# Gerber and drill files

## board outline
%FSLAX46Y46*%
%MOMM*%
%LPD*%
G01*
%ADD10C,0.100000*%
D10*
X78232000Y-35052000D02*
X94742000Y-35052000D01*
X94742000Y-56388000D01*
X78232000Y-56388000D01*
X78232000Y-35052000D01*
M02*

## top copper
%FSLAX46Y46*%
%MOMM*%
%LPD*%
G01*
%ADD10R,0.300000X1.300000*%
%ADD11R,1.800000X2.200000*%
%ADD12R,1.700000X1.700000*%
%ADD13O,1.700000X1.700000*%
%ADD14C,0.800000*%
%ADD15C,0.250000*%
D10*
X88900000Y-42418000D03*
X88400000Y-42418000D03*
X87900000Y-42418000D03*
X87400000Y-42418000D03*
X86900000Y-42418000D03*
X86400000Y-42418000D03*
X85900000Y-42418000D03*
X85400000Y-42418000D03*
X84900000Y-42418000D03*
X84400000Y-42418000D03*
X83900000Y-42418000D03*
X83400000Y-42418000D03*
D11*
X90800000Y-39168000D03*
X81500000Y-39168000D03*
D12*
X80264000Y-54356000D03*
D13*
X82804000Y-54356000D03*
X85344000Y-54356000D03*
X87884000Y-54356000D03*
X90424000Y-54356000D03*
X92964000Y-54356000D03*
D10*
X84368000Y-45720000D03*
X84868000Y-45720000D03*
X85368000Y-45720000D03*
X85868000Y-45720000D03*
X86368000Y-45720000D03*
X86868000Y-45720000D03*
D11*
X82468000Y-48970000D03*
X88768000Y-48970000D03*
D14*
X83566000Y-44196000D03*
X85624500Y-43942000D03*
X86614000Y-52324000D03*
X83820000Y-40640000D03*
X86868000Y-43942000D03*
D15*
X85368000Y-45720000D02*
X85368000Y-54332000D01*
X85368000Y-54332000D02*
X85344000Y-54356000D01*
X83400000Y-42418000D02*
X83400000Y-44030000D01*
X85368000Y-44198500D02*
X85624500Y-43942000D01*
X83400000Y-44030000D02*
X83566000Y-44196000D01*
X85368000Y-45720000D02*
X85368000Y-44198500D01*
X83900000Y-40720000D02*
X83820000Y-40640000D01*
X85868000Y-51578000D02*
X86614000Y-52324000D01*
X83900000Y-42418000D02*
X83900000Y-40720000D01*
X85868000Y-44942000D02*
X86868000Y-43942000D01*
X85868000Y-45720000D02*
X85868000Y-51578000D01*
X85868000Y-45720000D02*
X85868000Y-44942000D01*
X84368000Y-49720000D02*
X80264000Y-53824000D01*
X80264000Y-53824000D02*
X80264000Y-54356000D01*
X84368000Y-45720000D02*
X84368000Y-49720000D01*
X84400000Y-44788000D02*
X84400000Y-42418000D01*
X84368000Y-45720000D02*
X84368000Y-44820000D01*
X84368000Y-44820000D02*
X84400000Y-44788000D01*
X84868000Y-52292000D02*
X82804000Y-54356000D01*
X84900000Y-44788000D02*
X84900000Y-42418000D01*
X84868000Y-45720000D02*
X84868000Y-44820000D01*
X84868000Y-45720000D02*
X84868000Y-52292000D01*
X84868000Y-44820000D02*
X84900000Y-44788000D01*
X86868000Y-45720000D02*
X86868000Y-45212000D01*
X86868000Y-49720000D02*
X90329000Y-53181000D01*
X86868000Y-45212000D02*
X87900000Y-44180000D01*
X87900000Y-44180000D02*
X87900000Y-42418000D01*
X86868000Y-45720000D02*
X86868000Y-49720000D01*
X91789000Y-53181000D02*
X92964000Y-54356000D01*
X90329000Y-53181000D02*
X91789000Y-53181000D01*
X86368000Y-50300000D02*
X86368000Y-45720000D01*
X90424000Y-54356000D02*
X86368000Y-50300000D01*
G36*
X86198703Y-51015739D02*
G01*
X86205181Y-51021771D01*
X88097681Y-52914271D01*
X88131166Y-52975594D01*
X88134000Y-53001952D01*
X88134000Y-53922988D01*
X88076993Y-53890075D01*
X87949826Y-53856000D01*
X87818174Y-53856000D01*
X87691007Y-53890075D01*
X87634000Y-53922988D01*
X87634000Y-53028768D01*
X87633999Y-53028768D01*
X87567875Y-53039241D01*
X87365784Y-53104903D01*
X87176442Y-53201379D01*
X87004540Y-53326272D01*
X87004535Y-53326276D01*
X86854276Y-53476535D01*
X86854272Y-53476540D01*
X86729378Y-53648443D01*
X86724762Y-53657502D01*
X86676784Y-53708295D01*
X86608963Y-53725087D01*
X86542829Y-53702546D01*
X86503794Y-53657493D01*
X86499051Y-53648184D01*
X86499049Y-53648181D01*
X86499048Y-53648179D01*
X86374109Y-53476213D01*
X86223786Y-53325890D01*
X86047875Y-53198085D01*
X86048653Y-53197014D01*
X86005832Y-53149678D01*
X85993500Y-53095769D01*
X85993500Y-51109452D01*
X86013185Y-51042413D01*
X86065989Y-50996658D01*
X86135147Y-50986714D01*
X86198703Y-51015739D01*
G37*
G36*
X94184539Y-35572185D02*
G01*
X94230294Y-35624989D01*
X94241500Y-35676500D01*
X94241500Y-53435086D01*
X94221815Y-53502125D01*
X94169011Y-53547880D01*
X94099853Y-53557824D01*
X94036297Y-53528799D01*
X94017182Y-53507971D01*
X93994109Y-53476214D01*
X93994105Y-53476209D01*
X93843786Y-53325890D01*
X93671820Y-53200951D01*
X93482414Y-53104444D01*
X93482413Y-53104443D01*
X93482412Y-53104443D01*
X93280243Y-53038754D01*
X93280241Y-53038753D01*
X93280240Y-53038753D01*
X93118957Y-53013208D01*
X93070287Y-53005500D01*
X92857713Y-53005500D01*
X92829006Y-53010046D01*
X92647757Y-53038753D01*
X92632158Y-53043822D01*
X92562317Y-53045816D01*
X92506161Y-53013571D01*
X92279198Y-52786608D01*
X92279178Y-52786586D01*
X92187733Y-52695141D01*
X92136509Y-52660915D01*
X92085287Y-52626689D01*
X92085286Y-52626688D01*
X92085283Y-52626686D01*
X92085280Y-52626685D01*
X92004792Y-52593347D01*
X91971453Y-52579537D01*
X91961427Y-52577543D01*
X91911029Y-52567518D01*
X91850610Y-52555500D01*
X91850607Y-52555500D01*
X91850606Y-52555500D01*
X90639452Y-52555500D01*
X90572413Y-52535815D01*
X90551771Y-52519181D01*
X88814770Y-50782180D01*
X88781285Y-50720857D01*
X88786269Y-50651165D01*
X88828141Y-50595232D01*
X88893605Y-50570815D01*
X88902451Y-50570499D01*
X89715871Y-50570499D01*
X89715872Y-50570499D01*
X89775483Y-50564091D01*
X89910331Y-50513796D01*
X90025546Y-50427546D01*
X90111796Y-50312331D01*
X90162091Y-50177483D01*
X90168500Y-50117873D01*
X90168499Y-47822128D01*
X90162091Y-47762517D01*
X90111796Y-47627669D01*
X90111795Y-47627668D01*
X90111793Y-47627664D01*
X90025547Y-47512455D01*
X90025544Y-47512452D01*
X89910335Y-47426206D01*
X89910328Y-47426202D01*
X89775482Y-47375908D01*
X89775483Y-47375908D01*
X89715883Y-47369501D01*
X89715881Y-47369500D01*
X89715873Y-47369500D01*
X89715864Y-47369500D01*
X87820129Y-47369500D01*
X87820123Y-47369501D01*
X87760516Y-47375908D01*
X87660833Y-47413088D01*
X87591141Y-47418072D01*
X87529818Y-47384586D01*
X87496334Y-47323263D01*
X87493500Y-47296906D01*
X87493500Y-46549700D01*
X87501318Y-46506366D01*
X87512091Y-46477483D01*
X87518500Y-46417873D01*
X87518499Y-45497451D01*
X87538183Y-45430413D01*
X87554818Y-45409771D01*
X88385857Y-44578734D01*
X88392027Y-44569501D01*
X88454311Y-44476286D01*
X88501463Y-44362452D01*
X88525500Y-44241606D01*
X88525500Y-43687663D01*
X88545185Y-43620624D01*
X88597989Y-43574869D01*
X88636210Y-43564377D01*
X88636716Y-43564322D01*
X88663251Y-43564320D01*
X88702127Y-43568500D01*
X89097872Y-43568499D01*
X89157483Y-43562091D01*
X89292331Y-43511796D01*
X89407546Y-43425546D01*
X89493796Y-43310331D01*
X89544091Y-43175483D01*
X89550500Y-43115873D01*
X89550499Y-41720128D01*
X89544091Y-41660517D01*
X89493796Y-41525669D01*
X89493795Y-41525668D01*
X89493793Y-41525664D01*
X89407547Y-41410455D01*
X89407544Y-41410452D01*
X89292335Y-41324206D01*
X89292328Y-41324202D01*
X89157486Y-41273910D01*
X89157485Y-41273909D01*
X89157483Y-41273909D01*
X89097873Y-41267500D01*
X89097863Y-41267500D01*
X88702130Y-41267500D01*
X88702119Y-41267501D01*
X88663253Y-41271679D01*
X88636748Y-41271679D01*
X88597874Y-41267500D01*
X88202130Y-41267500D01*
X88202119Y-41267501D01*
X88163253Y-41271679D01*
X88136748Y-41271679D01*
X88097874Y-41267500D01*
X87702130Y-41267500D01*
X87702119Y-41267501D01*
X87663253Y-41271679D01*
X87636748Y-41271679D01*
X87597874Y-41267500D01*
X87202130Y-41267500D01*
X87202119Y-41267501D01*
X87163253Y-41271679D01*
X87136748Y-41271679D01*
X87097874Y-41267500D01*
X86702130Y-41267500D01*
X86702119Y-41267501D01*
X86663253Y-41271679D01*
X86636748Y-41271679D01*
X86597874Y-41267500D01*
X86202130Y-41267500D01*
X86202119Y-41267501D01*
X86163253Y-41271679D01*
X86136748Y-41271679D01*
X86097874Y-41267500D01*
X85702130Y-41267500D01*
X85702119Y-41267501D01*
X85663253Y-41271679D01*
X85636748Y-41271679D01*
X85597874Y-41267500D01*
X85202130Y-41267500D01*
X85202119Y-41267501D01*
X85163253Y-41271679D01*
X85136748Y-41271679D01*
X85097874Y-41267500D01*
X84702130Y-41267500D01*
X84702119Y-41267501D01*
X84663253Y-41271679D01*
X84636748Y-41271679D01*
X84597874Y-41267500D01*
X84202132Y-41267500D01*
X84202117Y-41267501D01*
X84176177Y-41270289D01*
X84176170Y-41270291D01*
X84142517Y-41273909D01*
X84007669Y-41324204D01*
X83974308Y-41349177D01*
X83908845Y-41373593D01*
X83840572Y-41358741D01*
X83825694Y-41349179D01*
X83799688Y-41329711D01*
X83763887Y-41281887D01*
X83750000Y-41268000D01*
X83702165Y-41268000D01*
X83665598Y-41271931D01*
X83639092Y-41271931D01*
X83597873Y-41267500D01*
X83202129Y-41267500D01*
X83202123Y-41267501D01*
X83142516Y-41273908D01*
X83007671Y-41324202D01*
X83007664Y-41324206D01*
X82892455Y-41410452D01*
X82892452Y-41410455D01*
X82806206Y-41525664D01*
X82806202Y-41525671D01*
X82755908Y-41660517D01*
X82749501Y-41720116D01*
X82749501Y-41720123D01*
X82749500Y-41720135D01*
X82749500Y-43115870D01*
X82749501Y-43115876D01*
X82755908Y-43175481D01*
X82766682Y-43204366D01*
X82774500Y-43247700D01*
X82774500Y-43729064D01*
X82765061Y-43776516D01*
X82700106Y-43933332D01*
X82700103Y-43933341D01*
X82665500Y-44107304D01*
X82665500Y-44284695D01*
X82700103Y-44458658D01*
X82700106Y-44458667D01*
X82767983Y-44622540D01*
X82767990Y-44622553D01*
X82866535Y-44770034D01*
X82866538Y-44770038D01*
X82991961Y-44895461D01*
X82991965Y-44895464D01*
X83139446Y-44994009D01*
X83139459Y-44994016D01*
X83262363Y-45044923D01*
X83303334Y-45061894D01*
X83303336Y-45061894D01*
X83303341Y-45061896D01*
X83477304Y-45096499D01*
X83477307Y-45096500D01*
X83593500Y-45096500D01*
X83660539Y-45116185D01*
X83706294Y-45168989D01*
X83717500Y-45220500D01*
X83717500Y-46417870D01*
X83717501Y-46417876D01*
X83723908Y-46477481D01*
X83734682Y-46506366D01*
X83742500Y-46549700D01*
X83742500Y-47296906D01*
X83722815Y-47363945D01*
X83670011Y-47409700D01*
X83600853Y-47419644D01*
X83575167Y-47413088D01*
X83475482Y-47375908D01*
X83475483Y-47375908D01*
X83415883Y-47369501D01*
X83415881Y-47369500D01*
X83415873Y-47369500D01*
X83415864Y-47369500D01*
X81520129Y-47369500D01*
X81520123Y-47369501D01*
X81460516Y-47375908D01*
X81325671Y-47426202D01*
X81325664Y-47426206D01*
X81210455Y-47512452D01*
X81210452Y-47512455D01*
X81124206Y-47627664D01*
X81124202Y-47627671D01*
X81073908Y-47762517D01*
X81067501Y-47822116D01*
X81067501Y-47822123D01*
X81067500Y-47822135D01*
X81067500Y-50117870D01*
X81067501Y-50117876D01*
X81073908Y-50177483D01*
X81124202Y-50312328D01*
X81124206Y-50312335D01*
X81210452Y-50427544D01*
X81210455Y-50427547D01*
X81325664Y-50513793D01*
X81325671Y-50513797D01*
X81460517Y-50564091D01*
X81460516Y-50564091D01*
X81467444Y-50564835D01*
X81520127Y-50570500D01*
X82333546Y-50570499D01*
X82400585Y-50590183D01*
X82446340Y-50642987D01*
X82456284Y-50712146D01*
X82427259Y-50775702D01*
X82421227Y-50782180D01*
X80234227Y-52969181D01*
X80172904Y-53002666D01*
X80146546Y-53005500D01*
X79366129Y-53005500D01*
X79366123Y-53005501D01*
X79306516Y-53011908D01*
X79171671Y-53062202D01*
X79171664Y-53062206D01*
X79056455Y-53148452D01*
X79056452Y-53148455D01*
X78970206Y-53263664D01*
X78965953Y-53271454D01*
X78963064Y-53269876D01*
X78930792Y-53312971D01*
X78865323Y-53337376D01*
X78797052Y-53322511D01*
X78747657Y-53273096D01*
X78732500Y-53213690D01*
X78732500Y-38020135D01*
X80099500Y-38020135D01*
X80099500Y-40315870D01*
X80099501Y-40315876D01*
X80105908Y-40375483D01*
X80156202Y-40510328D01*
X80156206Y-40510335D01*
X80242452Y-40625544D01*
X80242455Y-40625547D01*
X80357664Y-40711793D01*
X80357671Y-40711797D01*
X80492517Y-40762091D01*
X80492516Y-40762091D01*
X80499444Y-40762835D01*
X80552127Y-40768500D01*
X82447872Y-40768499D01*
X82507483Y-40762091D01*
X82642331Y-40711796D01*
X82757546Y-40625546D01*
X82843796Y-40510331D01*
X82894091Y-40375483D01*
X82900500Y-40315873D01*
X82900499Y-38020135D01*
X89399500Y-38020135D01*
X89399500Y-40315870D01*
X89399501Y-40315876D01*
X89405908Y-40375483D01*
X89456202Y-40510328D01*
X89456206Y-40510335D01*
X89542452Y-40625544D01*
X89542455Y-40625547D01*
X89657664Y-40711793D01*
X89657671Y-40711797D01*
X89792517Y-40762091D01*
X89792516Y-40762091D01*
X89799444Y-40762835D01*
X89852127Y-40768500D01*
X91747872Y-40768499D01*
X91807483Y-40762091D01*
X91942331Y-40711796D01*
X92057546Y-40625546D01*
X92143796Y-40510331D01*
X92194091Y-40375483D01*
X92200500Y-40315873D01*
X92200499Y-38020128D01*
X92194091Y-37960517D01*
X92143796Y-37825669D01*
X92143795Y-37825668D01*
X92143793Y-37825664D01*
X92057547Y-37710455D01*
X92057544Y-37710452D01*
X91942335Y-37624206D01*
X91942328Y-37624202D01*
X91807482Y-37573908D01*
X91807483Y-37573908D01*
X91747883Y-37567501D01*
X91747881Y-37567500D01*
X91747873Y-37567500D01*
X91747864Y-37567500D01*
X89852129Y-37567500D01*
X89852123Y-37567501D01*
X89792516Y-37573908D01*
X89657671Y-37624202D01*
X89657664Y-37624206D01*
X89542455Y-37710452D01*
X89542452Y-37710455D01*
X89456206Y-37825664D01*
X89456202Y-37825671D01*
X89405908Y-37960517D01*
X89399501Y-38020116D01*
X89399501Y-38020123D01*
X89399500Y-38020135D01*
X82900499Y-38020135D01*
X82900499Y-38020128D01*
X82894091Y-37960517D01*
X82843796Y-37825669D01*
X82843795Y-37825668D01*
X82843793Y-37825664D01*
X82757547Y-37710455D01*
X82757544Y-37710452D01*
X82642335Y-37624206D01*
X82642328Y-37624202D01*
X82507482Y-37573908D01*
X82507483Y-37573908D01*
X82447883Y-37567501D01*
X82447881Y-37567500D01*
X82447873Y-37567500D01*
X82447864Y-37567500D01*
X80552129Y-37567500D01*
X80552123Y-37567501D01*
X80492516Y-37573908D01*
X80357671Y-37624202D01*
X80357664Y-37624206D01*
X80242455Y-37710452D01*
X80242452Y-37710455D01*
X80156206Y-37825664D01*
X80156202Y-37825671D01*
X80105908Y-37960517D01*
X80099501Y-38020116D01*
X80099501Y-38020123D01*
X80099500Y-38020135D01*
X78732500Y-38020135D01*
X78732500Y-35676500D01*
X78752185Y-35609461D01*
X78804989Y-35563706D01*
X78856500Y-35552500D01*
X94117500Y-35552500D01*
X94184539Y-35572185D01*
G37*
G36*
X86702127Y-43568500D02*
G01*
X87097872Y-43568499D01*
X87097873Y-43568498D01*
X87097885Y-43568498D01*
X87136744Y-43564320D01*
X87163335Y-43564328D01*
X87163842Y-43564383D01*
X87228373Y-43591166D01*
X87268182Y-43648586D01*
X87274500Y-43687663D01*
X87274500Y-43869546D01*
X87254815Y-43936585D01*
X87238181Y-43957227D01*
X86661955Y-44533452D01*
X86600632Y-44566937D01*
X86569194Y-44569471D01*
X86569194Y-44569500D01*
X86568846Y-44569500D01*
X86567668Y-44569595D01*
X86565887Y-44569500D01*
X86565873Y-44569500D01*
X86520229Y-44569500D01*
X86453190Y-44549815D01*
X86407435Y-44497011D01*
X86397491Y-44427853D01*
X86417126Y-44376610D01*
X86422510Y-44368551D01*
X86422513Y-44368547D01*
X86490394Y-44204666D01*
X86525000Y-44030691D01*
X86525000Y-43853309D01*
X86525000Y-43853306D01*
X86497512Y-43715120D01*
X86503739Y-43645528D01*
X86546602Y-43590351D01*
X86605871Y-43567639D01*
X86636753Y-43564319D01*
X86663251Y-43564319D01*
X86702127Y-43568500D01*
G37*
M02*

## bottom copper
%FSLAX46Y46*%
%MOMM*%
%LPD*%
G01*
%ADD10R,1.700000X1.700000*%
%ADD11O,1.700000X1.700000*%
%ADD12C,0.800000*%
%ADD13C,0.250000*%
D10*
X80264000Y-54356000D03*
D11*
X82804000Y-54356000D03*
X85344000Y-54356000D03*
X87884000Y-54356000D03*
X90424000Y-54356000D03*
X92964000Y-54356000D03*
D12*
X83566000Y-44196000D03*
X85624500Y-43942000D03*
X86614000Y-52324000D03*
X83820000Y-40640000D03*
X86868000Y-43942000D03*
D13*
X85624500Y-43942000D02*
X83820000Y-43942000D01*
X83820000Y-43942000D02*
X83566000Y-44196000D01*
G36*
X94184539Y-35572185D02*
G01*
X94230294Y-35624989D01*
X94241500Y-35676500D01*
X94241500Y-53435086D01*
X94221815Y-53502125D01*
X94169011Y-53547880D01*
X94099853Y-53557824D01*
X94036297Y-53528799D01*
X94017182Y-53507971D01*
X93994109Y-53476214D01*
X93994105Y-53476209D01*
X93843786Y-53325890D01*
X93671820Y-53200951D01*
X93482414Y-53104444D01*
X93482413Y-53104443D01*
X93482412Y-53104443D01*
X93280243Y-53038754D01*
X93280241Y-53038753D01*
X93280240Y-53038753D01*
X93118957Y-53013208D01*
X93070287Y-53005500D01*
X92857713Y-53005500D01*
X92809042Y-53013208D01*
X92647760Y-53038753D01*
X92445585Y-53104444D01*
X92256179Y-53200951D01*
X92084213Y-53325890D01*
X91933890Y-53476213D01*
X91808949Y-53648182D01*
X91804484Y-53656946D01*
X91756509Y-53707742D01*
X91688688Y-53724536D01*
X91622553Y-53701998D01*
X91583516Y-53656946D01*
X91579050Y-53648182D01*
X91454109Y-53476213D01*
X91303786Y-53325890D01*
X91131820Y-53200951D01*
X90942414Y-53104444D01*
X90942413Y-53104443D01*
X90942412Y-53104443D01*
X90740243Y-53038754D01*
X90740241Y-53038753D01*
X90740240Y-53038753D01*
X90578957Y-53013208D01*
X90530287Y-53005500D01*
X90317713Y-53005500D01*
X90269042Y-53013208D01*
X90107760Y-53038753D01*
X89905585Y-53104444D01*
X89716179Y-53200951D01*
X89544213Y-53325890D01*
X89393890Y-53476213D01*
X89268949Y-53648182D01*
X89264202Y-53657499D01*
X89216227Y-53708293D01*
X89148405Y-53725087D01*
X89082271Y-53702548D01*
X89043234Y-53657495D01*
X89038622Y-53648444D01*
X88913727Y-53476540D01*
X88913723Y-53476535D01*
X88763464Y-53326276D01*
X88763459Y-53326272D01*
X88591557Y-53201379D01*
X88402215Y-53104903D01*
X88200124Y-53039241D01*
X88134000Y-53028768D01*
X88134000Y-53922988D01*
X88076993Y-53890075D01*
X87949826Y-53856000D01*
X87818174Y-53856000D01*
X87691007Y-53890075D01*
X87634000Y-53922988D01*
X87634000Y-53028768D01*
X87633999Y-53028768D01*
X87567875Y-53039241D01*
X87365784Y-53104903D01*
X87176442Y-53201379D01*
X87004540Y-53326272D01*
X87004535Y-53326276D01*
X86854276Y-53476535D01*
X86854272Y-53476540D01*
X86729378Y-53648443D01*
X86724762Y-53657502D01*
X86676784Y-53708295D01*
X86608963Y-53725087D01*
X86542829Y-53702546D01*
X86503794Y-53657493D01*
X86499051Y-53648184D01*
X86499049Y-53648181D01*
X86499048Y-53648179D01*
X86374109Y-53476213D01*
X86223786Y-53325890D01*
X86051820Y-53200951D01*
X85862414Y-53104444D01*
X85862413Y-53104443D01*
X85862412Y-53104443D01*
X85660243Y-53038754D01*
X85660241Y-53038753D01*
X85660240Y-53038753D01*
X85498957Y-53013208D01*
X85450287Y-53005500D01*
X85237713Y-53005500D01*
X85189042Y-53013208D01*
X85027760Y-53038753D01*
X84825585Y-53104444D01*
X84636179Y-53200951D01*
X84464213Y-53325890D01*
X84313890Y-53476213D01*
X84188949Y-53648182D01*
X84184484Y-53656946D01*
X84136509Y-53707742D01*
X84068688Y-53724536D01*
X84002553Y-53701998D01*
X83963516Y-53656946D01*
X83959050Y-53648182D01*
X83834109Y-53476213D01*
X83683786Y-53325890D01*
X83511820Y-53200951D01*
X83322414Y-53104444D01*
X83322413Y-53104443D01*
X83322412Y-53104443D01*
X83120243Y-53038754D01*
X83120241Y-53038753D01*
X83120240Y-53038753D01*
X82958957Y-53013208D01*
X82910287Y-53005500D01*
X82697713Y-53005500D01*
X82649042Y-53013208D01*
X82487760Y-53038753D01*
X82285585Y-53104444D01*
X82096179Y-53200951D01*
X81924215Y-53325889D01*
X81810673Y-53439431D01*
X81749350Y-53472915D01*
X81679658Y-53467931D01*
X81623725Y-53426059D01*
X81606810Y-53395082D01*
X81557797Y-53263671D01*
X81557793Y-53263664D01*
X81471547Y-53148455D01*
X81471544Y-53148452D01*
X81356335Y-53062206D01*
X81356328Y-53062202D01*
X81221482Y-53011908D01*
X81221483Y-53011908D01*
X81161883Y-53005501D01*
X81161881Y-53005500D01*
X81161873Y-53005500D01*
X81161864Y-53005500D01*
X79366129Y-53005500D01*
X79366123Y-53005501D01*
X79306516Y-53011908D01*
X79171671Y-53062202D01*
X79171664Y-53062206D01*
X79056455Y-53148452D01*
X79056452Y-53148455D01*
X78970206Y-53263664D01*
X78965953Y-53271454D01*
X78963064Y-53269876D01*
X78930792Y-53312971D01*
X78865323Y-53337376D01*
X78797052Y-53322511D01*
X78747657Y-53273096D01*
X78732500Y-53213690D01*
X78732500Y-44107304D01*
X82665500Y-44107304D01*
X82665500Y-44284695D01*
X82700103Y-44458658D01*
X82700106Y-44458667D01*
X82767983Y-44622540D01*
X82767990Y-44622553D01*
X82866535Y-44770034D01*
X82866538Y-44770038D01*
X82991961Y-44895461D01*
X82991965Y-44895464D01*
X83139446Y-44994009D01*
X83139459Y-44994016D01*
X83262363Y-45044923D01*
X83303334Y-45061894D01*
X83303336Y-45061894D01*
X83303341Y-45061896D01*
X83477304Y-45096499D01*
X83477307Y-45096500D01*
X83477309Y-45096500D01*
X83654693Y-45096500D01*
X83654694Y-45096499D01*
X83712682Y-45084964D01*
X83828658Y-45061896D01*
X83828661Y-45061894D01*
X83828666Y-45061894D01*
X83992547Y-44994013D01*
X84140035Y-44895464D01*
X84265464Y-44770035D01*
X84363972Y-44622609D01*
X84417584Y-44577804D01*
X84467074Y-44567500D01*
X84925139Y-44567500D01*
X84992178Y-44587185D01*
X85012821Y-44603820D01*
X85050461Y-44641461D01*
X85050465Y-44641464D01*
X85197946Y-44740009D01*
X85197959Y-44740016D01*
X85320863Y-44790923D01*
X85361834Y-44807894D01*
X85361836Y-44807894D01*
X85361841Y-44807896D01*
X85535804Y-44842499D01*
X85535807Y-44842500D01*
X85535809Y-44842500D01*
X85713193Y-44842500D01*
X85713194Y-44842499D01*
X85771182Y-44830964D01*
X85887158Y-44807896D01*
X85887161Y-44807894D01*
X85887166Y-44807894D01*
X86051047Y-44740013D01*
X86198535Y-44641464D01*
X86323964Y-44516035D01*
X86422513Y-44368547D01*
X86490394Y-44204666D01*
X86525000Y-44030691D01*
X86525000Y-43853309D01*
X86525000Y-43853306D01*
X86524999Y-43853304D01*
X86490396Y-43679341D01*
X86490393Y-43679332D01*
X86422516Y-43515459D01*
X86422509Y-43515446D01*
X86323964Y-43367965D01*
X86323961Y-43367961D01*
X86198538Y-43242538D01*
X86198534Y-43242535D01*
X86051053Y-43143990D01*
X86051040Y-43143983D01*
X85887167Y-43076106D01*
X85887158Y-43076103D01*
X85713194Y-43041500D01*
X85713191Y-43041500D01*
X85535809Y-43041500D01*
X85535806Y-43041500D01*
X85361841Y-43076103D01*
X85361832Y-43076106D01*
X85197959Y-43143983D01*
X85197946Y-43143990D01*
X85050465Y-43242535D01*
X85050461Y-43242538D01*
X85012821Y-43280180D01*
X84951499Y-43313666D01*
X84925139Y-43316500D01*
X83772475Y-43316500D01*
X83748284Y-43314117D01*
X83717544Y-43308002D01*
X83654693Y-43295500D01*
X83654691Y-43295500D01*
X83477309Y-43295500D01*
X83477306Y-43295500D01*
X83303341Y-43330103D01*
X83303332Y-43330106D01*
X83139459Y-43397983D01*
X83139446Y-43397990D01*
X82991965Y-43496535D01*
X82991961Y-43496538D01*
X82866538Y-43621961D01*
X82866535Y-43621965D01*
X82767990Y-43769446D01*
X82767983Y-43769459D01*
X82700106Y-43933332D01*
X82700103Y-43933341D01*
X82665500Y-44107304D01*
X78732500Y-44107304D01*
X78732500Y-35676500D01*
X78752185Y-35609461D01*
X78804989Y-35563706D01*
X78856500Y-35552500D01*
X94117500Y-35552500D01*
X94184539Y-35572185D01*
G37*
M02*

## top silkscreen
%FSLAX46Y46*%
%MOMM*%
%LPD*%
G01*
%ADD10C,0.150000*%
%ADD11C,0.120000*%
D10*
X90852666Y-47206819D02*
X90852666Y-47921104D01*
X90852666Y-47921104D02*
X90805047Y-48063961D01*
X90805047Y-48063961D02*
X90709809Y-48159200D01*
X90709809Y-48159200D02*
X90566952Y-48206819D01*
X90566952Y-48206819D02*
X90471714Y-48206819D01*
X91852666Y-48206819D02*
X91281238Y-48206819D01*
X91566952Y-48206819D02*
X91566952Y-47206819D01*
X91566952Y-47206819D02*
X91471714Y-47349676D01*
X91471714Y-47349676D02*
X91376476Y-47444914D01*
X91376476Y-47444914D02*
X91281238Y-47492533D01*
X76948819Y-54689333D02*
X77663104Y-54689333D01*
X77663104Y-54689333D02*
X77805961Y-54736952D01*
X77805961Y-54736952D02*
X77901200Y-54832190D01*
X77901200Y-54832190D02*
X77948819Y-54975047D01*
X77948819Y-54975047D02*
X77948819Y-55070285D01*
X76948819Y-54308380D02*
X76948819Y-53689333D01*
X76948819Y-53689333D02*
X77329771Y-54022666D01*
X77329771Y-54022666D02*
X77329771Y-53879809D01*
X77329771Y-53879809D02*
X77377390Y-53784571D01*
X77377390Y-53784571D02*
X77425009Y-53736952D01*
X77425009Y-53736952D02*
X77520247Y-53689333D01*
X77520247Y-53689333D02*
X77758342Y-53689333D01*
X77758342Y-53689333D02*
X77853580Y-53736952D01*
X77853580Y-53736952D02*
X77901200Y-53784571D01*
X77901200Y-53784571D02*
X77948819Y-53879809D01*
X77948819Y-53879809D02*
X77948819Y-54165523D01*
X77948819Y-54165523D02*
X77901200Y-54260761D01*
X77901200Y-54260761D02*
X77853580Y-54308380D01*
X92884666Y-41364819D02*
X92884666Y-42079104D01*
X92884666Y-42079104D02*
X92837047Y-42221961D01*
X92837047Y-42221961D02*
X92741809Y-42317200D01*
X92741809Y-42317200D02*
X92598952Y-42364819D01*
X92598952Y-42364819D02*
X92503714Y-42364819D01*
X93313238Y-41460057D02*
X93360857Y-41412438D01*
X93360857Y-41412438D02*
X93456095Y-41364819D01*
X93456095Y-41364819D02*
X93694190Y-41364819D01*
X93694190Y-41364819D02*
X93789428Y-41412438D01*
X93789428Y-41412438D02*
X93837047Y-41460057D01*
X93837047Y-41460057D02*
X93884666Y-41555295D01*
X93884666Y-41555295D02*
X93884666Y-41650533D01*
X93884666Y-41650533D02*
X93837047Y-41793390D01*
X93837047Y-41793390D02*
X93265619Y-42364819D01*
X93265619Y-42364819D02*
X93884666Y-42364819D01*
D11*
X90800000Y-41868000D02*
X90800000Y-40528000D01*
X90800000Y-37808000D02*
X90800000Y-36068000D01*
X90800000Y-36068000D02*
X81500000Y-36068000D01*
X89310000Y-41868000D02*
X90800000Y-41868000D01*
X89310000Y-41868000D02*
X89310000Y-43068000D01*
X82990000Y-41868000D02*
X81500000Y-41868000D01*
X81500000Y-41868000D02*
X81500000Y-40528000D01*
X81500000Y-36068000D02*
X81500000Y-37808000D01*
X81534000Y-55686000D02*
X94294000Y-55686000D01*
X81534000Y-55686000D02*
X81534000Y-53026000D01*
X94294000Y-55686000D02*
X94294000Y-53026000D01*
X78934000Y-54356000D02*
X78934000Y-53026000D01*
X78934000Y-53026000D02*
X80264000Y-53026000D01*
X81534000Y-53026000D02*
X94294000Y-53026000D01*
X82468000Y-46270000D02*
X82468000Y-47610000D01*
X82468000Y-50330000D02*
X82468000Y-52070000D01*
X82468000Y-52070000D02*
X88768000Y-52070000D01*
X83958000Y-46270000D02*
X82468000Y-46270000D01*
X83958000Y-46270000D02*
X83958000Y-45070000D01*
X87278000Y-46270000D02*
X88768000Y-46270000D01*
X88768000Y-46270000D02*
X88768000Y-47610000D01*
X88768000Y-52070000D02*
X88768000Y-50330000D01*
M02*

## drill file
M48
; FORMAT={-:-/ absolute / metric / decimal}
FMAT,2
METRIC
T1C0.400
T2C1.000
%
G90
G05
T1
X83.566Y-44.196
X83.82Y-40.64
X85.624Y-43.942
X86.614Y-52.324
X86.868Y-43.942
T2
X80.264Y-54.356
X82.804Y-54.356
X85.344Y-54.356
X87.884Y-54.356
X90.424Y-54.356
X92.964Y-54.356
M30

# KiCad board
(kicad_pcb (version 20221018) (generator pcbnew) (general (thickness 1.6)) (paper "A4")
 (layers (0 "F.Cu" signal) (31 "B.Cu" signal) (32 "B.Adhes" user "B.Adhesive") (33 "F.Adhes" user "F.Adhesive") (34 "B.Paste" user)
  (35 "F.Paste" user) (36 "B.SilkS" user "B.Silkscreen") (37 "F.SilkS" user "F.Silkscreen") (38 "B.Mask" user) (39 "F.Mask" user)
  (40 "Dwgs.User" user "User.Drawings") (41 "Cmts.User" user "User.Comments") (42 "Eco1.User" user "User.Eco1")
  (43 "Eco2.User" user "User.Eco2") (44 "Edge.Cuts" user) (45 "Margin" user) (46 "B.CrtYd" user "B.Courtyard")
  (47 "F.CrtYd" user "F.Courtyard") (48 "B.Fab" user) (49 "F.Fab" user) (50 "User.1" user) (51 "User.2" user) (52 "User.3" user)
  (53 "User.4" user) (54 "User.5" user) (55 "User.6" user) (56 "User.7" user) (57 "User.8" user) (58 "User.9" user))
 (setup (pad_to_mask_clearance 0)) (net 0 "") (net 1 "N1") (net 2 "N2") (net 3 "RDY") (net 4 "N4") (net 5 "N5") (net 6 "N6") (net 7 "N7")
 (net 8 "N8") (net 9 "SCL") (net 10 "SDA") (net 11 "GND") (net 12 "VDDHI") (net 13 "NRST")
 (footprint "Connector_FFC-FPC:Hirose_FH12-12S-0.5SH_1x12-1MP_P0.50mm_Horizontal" (layer "F.Cu") (at 86.15 40.568 180)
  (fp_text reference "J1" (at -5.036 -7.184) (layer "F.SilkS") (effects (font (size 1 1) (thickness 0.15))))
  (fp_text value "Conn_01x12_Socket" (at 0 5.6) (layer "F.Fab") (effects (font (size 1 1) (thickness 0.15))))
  (fp_line (start -4.65 -1.3) (end -4.65 0.04) (stroke (width 0.12) (type solid)) (layer "F.SilkS"))
  (fp_line (start -4.65 2.76) (end -4.65 4.5) (stroke (width 0.12) (type solid)) (layer "F.SilkS"))
  (fp_line (start -4.65 4.5) (end 4.65 4.5) (stroke (width 0.12) (type solid)) (layer "F.SilkS"))
  (fp_line (start -3.16 -1.3) (end -4.65 -1.3) (stroke (width 0.12) (type solid)) (layer "F.SilkS"))
  (fp_line (start -3.16 -1.3) (end -3.16 -2.5) (stroke (width 0.12) (type solid)) (layer "F.SilkS"))
  (fp_line (start 3.16 -1.3) (end 4.65 -1.3) (stroke (width 0.12) (type solid)) (layer "F.SilkS"))
  (fp_line (start 4.65 -1.3) (end 4.65 0.04) (stroke (width 0.12) (type solid)) (layer "F.SilkS"))
  (fp_line (start 4.65 4.5) (end 4.65 2.76) (stroke (width 0.12) (type solid)) (layer "F.SilkS"))
  (pad "1" smd rect (at -2.75 -1.85 180) (size 0.3 1.3) (layers "F.Cu" "F.Paste" "F.Mask") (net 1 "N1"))
  (pad "2" smd rect (at -2.25 -1.85 180) (size 0.3 1.3) (layers "F.Cu" "F.Paste" "F.Mask") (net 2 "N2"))
  (pad "3" smd rect (at -1.75 -1.85 180) (size 0.3 1.3) (layers "F.Cu" "F.Paste" "F.Mask") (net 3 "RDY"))
  (pad "4" smd rect (at -1.25 -1.85 180) (size 0.3 1.3) (layers "F.Cu" "F.Paste" "F.Mask") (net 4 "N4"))
  (pad "5" smd rect (at -0.75 -1.85 180) (size 0.3 1.3) (layers "F.Cu" "F.Paste" "F.Mask") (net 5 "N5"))
  (pad "6" smd rect (at -0.25 -1.85 180) (size 0.3 1.3) (layers "F.Cu" "F.Paste" "F.Mask") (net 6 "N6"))
  (pad "7" smd rect (at 0.25 -1.85 180) (size 0.3 1.3) (layers "F.Cu" "F.Paste" "F.Mask") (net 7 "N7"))
  (pad "8" smd rect (at 0.75 -1.85 180) (size 0.3 1.3) (layers "F.Cu" "F.Paste" "F.Mask") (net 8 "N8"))
  (pad "9" smd rect (at 1.25 -1.85 180) (size 0.3 1.3) (layers "F.Cu" "F.Paste" "F.Mask") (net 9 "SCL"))
  (pad "10" smd rect (at 1.75 -1.85 180) (size 0.3 1.3) (layers "F.Cu" "F.Paste" "F.Mask") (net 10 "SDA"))
  (pad "11" smd rect (at 2.25 -1.85 180) (size 0.3 1.3) (layers "F.Cu" "F.Paste" "F.Mask") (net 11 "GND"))
  (pad "12" smd rect (at 2.75 -1.85 180) (size 0.3 1.3) (layers "F.Cu" "F.Paste" "F.Mask") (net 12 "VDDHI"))
  (pad "MP" smd rect (at -4.65 1.4 180) (size 1.8 2.2) (layers "F.Cu" "F.Paste" "F.Mask"))
  (pad "MP" smd rect (at 4.65 1.4 180) (size 1.8 2.2) (layers "F.Cu" "F.Paste" "F.Mask")))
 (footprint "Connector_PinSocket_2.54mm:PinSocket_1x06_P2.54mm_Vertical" (layer "F.Cu") (at 80.264 54.356 90)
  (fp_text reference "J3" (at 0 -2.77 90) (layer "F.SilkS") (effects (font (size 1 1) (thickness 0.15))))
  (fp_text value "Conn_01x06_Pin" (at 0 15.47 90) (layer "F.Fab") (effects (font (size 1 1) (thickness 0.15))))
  (fp_line (start -1.33 1.27) (end -1.33 14.03) (stroke (width 0.12) (type solid)) (layer "F.SilkS"))
  (fp_line (start -1.33 1.27) (end 1.33 1.27) (stroke (width 0.12) (type solid)) (layer "F.SilkS"))
  (fp_line (start -1.33 14.03) (end 1.33 14.03) (stroke (width 0.12) (type solid)) (layer "F.SilkS"))
  (fp_line (start 0 -1.33) (end 1.33 -1.33) (stroke (width 0.12) (type solid)) (layer "F.SilkS"))
  (fp_line (start 1.33 -1.33) (end 1.33 0) (stroke (width 0.12) (type solid)) (layer "F.SilkS"))
  (fp_line (start 1.33 1.27) (end 1.33 14.03) (stroke (width 0.12) (type solid)) (layer "F.SilkS"))
  (pad "1" thru_hole rect (at 0 0 90) (size 1.7 1.7) (drill 1) (layers "*.Cu" "*.Mask") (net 10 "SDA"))
  (pad "2" thru_hole oval (at 0 2.54 90) (size 1.7 1.7) (drill 1) (layers "*.Cu" "*.Mask") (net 9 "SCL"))
  (pad "3" thru_hole oval (at 0 5.08 90) (size 1.7 1.7) (drill 1) (layers "*.Cu" "*.Mask") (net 12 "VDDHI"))
  (pad "4" thru_hole oval (at 0 7.62 90) (size 1.7 1.7) (drill 1) (layers "*.Cu" "*.Mask") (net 11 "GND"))
  (pad "5" thru_hole oval (at 0 10.16 90) (size 1.7 1.7) (drill 1) (layers "*.Cu" "*.Mask") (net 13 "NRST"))
  (pad "6" thru_hole oval (at 0 12.7 90) (size 1.7 1.7) (drill 1) (layers "*.Cu" "*.Mask") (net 3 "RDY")))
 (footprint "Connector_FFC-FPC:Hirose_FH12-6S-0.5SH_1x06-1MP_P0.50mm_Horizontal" (layer "F.Cu") (at 85.618 47.57)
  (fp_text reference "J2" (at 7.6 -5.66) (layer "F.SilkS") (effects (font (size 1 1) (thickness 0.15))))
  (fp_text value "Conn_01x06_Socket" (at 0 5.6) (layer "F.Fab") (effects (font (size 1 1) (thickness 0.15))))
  (fp_line (start -3.15 -1.3) (end -3.15 0.04) (stroke (width 0.12) (type solid)) (layer "F.SilkS"))
  (fp_line (start -3.15 2.76) (end -3.15 4.5) (stroke (width 0.12) (type solid)) (layer "F.SilkS"))
  (fp_line (start -3.15 4.5) (end 3.15 4.5) (stroke (width 0.12) (type solid)) (layer "F.SilkS"))
  (fp_line (start -1.66 -1.3) (end -3.15 -1.3) (stroke (width 0.12) (type solid)) (layer "F.SilkS"))
  (fp_line (start -1.66 -1.3) (end -1.66 -2.5) (stroke (width 0.12) (type solid)) (layer "F.SilkS"))
  (fp_line (start 1.66 -1.3) (end 3.15 -1.3) (stroke (width 0.12) (type solid)) (layer "F.SilkS"))
  (fp_line (start 3.15 -1.3) (end 3.15 0.04) (stroke (width 0.12) (type solid)) (layer "F.SilkS"))
  (fp_line (start 3.15 4.5) (end 3.15 2.76) (stroke (width 0.12) (type solid)) (layer "F.SilkS"))
  (pad "1" smd rect (at -1.25 -1.85) (size 0.3 1.3) (layers "F.Cu" "F.Paste" "F.Mask") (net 10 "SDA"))
  (pad "2" smd rect (at -0.75 -1.85) (size 0.3 1.3) (layers "F.Cu" "F.Paste" "F.Mask") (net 9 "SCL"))
  (pad "3" smd rect (at -0.25 -1.85) (size 0.3 1.3) (layers "F.Cu" "F.Paste" "F.Mask") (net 12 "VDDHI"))
  (pad "4" smd rect (at 0.25 -1.85) (size 0.3 1.3) (layers "F.Cu" "F.Paste" "F.Mask") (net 11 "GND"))
  (pad "5" smd rect (at 0.75 -1.85) (size 0.3 1.3) (layers "F.Cu" "F.Paste" "F.Mask") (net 13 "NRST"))
  (pad "6" smd rect (at 1.25 -1.85) (size 0.3 1.3) (layers "F.Cu" "F.Paste" "F.Mask") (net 3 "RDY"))
  (pad "MP" smd rect (at -3.15 1.4) (size 1.8 2.2) (layers "F.Cu" "F.Paste" "F.Mask"))
  (pad "MP" smd rect (at 3.15 1.4) (size 1.8 2.2) (layers "F.Cu" "F.Paste" "F.Mask")))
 (gr_rect (start 78.232 35.052) (end 94.742 56.388) (stroke (width 0.1) (type default)) (fill none) (layer "Edge.Cuts"))
 (segment (start 85.368 45.72) (end 85.368 54.332) (width 0.25) (layer "F.Cu") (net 12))
 (segment (start 85.368 54.332) (end 85.344 54.356) (width 0.25) (layer "F.Cu") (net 12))
 (segment (start 83.4 42.418) (end 83.4 44.03) (width 0.25) (layer "F.Cu") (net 12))
 (segment (start 85.368 44.1985) (end 85.6245 43.942) (width 0.25) (layer "F.Cu") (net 12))
 (segment (start 83.4 44.03) (end 83.566 44.196) (width 0.25) (layer "F.Cu") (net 12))
 (segment (start 85.368 45.72) (end 85.368 44.1985) (width 0.25) (layer "F.Cu") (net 12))
 (via (at 83.566 44.196) (size 0.8) (drill 0.4) (layers "F.Cu" "B.Cu") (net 12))
 (via (at 85.6245 43.942) (size 0.8) (drill 0.4) (layers "F.Cu" "B.Cu") (free) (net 12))
 (segment (start 85.6245 43.942) (end 83.82 43.942) (width 0.25) (layer "B.Cu") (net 12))
 (segment (start 83.82 43.942) (end 83.566 44.196) (width 0.25) (layer "B.Cu") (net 12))
 (segment (start 83.9 40.72) (end 83.82 40.64) (width 0.25) (layer "F.Cu") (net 11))
 (segment (start 85.868 51.578) (end 86.614 52.324) (width 0.25) (layer "F.Cu") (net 11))
 (segment (start 83.9 42.418) (end 83.9 40.72) (width 0.25) (layer "F.Cu") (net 11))
 (segment (start 85.868 44.942) (end 86.868 43.942) (width 0.25) (layer "F.Cu") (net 11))
 (segment (start 85.868 45.72) (end 85.868 51.578) (width 0.25) (layer "F.Cu") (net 11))
 (segment (start 85.868 45.72) (end 85.868 44.942) (width 0.25) (layer "F.Cu") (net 11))
 (via (at 86.614 52.324) (size 0.8) (drill 0.4) (layers "F.Cu" "B.Cu") (free) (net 11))
 (via (at 83.82 40.64) (size 0.8) (drill 0.4) (layers "F.Cu" "B.Cu") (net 11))
 (via (at 86.868 43.942) (size 0.8) (drill 0.4) (layers "F.Cu" "B.Cu") (free) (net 11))
 (segment (start 84.368 49.72) (end 80.264 53.824) (width 0.25) (layer "F.Cu") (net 10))
 (segment (start 80.264 53.824) (end 80.264 54.356) (width 0.25) (layer "F.Cu") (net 10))
 (segment (start 84.368 45.72) (end 84.368 49.72) (width 0.25) (layer "F.Cu") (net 10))
 (segment (start 84.4 44.788) (end 84.4 42.418) (width 0.25) (layer "F.Cu") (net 10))
 (segment (start 84.368 45.72) (end 84.368 44.82) (width 0.25) (layer "F.Cu") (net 10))
 (segment (start 84.368 44.82) (end 84.4 44.788) (width 0.25) (layer "F.Cu") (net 10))
 (segment (start 84.868 52.292) (end 82.804 54.356) (width 0.25) (layer "F.Cu") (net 9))
 (segment (start 84.9 44.788) (end 84.9 42.418) (width 0.25) (layer "F.Cu") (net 9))
 (segment (start 84.868 45.72) (end 84.868 44.82) (width 0.25) (layer "F.Cu") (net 9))
 (segment (start 84.868 45.72) (end 84.868 52.292) (width 0.25) (layer "F.Cu") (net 9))
 (segment (start 84.868 44.82) (end 84.9 44.788) (width 0.25) (layer "F.Cu") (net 9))
 (segment (start 86.868 45.72) (end 86.868 45.212) (width 0.25) (layer "F.Cu") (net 3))
 (segment (start 86.868 49.72) (end 90.329 53.181) (width 0.25) (layer "F.Cu") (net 3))
 (segment (start 86.868 45.212) (end 87.9 44.18) (width 0.25) (layer "F.Cu") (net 3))
 (segment (start 87.9 44.18) (end 87.9 42.418) (width 0.25) (layer "F.Cu") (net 3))
 (segment (start 86.868 45.72) (end 86.868 49.72) (width 0.25) (layer "F.Cu") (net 3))
 (segment (start 91.789 53.181) (end 92.964 54.356) (width 0.25) (layer "F.Cu") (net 3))
 (segment (start 90.329 53.181) (end 91.789 53.181) (width 0.25) (layer "F.Cu") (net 3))
 (segment (start 86.368 50.3) (end 86.368 45.72) (width 0.25) (layer "F.Cu") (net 13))
 (segment (start 90.424 54.356) (end 86.368 50.3) (width 0.25) (layer "F.Cu") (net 13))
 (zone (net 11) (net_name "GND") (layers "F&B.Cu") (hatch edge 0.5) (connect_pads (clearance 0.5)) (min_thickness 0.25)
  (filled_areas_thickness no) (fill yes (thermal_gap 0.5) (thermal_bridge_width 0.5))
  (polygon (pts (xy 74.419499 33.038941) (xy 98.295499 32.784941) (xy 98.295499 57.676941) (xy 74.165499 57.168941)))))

